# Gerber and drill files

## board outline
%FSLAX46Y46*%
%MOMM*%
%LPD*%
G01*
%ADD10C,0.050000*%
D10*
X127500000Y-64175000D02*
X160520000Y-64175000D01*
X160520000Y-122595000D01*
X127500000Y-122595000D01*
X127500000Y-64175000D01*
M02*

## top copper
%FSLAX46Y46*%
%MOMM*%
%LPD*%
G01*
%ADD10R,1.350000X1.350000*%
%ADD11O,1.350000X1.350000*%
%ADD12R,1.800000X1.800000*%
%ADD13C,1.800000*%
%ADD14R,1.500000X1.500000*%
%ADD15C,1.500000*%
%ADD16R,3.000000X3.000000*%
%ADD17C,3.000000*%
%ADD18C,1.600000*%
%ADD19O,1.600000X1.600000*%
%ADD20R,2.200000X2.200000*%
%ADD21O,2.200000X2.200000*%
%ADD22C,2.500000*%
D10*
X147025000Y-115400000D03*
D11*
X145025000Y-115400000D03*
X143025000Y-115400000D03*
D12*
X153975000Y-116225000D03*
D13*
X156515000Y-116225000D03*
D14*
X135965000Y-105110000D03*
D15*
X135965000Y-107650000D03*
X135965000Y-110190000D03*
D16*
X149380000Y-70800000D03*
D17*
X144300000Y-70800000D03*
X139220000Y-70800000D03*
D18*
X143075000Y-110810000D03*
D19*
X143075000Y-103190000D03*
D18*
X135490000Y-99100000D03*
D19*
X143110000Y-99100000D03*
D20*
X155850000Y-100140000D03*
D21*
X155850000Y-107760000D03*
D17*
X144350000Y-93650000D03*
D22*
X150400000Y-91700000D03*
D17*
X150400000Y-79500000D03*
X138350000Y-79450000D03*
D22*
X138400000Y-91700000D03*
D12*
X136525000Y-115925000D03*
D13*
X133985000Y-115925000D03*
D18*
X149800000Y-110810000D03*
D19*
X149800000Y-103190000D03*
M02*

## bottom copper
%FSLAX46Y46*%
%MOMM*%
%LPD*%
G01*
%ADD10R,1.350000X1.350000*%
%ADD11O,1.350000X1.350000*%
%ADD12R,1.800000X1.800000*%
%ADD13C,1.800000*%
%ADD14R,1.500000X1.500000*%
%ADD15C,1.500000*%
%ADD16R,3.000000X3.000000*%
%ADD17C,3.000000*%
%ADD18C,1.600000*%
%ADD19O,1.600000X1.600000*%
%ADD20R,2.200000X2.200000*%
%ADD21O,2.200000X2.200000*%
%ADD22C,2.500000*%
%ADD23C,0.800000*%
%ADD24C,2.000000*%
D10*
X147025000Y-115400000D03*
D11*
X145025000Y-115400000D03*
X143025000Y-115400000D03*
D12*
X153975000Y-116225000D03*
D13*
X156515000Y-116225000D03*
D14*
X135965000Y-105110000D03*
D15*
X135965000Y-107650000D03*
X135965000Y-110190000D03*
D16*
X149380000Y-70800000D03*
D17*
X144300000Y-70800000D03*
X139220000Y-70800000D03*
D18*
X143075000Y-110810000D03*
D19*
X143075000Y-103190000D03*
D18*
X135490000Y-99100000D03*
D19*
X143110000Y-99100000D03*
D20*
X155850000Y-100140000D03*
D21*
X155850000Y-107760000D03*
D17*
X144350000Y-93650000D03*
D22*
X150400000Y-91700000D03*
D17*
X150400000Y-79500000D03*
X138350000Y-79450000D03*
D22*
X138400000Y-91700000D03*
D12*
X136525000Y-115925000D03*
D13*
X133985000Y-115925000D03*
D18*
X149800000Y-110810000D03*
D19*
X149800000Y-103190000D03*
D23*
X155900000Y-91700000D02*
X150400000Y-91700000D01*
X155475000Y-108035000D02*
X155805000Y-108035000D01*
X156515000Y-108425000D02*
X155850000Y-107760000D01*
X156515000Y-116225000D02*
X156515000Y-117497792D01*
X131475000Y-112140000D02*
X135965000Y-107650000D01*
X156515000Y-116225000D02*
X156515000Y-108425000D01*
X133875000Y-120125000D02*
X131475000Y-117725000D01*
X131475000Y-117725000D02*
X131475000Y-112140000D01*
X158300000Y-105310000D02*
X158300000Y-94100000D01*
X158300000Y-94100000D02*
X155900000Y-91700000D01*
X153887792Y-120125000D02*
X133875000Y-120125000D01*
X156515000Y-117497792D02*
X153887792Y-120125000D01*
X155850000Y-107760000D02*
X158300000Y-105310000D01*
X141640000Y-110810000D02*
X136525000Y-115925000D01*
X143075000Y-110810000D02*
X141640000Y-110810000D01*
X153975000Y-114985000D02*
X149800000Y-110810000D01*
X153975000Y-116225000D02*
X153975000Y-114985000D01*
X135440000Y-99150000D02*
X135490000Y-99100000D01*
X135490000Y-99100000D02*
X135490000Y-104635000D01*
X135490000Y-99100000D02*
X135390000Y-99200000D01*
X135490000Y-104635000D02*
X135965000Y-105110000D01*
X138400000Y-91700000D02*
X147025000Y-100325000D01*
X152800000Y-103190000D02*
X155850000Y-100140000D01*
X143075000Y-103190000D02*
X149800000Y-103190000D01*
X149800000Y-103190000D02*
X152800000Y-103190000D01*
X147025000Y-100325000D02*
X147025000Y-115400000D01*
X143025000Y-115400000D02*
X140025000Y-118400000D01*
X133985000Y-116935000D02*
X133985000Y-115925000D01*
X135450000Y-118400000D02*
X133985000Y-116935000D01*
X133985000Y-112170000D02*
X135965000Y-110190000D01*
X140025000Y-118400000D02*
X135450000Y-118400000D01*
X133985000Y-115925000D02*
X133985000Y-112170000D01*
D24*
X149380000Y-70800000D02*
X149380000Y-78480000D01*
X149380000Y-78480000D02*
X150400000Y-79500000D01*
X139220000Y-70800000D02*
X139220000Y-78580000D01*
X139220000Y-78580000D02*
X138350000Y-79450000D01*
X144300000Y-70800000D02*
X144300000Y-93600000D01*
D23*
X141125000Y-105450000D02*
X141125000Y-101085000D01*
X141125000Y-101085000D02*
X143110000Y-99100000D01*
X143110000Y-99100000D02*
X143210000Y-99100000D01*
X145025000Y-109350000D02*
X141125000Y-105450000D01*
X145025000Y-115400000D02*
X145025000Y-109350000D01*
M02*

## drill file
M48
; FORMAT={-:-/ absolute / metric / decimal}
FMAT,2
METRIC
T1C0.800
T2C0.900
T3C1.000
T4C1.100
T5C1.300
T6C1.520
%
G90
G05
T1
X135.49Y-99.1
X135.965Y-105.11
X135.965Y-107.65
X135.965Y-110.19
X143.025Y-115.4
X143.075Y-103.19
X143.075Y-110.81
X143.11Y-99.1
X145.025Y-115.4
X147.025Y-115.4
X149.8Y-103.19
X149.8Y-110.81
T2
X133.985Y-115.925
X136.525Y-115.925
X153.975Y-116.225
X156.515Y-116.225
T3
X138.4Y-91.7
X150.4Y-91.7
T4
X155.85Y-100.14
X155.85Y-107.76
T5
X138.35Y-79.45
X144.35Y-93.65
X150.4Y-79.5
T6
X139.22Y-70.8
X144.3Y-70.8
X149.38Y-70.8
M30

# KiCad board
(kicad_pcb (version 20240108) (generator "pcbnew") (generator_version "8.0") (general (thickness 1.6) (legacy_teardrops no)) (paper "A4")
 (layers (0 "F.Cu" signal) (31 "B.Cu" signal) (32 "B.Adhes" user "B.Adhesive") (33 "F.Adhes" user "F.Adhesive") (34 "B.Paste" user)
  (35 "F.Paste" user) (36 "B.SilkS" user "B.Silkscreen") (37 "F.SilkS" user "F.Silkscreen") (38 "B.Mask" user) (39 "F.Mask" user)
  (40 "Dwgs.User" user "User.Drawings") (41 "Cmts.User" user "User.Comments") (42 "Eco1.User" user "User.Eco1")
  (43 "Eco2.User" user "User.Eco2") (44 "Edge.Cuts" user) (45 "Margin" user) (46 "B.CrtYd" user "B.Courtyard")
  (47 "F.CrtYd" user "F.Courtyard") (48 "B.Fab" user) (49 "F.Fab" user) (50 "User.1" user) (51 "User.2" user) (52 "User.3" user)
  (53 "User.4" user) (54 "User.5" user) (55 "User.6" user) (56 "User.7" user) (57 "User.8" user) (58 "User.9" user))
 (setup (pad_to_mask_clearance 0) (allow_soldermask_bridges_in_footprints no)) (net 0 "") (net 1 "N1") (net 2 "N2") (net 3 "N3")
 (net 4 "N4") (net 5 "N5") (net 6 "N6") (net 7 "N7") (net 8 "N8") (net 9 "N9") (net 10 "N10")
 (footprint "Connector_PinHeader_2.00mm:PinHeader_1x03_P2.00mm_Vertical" (layer "F.Cu") (at 147.025 115.4 -90)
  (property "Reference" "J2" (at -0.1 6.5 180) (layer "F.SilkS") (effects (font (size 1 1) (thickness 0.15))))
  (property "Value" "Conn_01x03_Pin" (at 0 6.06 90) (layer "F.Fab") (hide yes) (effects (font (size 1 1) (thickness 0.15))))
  (pad "1" thru_hole rect (at 0 0 270) (size 1.35 1.35) (drill 0.8) (layers "*.Cu" "*.Mask") (remove_unused_layers no) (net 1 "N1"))
  (pad "2" thru_hole oval (at 0 2 270) (size 1.35 1.35) (drill 0.8) (layers "*.Cu" "*.Mask") (remove_unused_layers no) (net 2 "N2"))
  (pad "3" thru_hole oval (at 0 4 270) (size 1.35 1.35) (drill 0.8) (layers "*.Cu" "*.Mask") (remove_unused_layers no) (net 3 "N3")))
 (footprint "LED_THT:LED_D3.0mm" (layer "F.Cu") (at 153.975 116.225)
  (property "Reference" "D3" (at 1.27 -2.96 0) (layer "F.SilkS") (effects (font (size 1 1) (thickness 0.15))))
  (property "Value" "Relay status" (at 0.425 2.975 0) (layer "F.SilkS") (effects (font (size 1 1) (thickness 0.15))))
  (pad "1" thru_hole rect (at 0 0) (size 1.8 1.8) (drill 0.9) (layers "*.Cu" "*.Mask") (remove_unused_layers no) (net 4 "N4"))
  (pad "2" thru_hole circle (at 2.54 0) (size 1.8 1.8) (drill 0.9) (layers "*.Cu" "*.Mask") (remove_unused_layers no) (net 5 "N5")))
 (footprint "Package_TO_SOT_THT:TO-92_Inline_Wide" (layer "F.Cu") (at 135.965 105.11 -90)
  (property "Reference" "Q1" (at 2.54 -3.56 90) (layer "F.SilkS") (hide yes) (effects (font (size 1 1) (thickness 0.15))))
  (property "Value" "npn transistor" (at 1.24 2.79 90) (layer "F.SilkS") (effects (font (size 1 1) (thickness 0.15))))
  (pad "1" thru_hole rect (at 0 0 270) (size 1.5 1.5) (drill 0.8) (layers "*.Cu" "*.Mask") (remove_unused_layers no) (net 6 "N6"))
  (pad "2" thru_hole circle (at 2.54 0 270) (size 1.5 1.5) (drill 0.8) (layers "*.Cu" "*.Mask") (remove_unused_layers no) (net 5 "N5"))
  (pad "3" thru_hole circle (at 5.08 0 270) (size 1.5 1.5) (drill 0.8) (layers "*.Cu" "*.Mask") (remove_unused_layers no) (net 3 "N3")))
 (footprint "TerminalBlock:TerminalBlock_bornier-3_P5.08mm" (layer "F.Cu") (at 149.38 70.8 180)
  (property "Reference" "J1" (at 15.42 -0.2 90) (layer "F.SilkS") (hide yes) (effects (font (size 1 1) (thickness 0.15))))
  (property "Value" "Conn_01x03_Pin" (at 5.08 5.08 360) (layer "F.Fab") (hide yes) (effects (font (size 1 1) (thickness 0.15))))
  (pad "1" thru_hole rect (at 0 0 180) (size 3 3) (drill 1.52) (layers "*.Cu" "*.Mask") (remove_unused_layers no) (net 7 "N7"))
  (pad "2" thru_hole circle (at 5.08 0 180) (size 3 3) (drill 1.52) (layers "*.Cu" "*.Mask") (remove_unused_layers no) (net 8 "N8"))
  (pad "3" thru_hole circle (at 10.16 0 180) (size 3 3) (drill 1.52) (layers "*.Cu" "*.Mask") (remove_unused_layers no) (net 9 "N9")))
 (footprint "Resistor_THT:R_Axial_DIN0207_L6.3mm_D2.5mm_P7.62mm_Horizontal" (layer "F.Cu") (at 143.075 110.81 90)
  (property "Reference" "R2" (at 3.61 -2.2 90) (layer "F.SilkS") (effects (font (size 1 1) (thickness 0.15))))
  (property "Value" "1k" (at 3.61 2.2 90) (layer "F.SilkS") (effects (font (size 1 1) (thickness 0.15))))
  (pad "1" thru_hole circle (at 0 0 90) (size 1.6 1.6) (drill 0.8) (layers "*.Cu" "*.Mask") (remove_unused_layers no) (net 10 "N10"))
  (pad "2" thru_hole oval (at 7.62 0 90) (size 1.6 1.6) (drill 0.8) (layers "*.Cu" "*.Mask") (remove_unused_layers no) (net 1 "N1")))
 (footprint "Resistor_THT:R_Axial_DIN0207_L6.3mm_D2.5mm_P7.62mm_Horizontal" (layer "F.Cu") (at 135.49 99.1)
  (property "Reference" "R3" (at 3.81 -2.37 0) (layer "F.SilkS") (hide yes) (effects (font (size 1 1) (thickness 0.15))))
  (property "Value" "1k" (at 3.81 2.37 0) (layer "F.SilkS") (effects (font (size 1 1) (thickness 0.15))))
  (pad "1" thru_hole circle (at 0 0) (size 1.6 1.6) (drill 0.8) (layers "*.Cu" "*.Mask") (remove_unused_layers no) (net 6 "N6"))
  (pad "2" thru_hole oval (at 7.62 0) (size 1.6 1.6) (drill 0.8) (layers "*.Cu" "*.Mask") (remove_unused_layers no) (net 2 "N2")))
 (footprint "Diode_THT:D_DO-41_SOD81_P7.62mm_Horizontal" (layer "F.Cu") (at 155.85 100.14 -90)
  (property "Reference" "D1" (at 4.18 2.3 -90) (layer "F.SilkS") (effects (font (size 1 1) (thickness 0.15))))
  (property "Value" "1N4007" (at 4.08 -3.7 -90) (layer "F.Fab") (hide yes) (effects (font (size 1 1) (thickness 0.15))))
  (pad "1" thru_hole rect (at 0 0 270) (size 2.2 2.2) (drill 1.1) (layers "*.Cu" "*.Mask") (remove_unused_layers no) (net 1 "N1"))
  (pad "2" thru_hole oval (at 7.62 0 270) (size 2.2 2.2) (drill 1.1) (layers "*.Cu" "*.Mask") (remove_unused_layers no) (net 5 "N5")))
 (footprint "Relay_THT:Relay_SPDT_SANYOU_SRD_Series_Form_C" (layer "F.Cu") (at 144.35 93.65 90)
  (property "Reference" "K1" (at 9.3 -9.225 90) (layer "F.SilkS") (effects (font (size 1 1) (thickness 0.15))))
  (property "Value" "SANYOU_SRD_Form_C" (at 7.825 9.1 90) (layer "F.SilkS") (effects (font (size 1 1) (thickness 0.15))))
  (pad "1" thru_hole circle (at 0 0 180) (size 3 3) (drill 1.3) (layers "*.Cu" "*.Mask") (remove_unused_layers no) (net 8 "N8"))
  (pad "2" thru_hole circle (at 1.95 6.05 180) (size 2.5 2.5) (drill 1) (layers "*.Cu" "*.Mask") (remove_unused_layers no) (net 5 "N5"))
  (pad "3" thru_hole circle (at 14.15 6.05 180) (size 3 3) (drill 1.3) (layers "*.Cu" "*.Mask") (remove_unused_layers no) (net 7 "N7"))
  (pad "4" thru_hole circle (at 14.2 -6 180) (size 3 3) (drill 1.3) (layers "*.Cu" "*.Mask") (remove_unused_layers no) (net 9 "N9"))
  (pad "5" thru_hole circle (at 1.95 -5.95 180) (size 2.5 2.5) (drill 1) (layers "*.Cu" "*.Mask") (remove_unused_layers no) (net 1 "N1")))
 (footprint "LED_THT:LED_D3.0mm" (layer "F.Cu") (at 136.525 115.925 180)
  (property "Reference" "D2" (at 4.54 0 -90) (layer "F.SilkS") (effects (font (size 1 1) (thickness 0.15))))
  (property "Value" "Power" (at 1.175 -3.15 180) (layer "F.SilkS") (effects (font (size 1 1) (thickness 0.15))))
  (pad "1" thru_hole rect (at 0 0 180) (size 1.8 1.8) (drill 0.9) (layers "*.Cu" "*.Mask") (remove_unused_layers no) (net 10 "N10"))
  (pad "2" thru_hole circle (at 2.54 0 180) (size 1.8 1.8) (drill 0.9) (layers "*.Cu" "*.Mask") (remove_unused_layers no) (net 3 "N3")))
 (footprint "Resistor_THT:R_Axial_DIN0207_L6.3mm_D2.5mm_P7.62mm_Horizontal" (layer "F.Cu") (at 149.8 110.81 90)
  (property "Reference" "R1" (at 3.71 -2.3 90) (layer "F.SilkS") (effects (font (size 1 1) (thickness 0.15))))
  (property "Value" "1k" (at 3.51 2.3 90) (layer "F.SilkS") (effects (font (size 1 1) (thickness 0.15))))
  (pad "1" thru_hole circle (at 0 0 90) (size 1.6 1.6) (drill 0.8) (layers "*.Cu" "*.Mask") (remove_unused_layers no) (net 4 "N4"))
  (pad "2" thru_hole oval (at 7.62 0 90) (size 1.6 1.6) (drill 0.8) (layers "*.Cu" "*.Mask") (remove_unused_layers no) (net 1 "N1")))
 (gr_rect (start 127.5 64.175) (end 160.52 122.595) (stroke (width 0.05) (type default)) (fill none) (layer "Edge.Cuts"))
 (segment (start 155.9 91.7) (end 150.4 91.7) (width 0.8) (layer "B.Cu") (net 5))
 (segment (start 155.475 108.035) (end 155.805 108.035) (width 0.8) (layer "B.Cu") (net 5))
 (segment (start 156.515 108.425) (end 155.85 107.76) (width 0.8) (layer "B.Cu") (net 5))
 (segment (start 156.515 116.225) (end 156.515 117.497792) (width 0.8) (layer "B.Cu") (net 5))
 (segment (start 131.475 112.14) (end 135.965 107.65) (width 0.8) (layer "B.Cu") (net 5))
 (segment (start 156.515 116.225) (end 156.515 108.425) (width 0.8) (layer "B.Cu") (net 5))
 (segment (start 133.875 120.125) (end 131.475 117.725) (width 0.8) (layer "B.Cu") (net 5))
 (segment (start 131.475 117.725) (end 131.475 112.14) (width 0.8) (layer "B.Cu") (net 5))
 (segment (start 158.3 105.31) (end 158.3 94.1) (width 0.8) (layer "B.Cu") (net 5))
 (segment (start 158.3 94.1) (end 155.9 91.7) (width 0.8) (layer "B.Cu") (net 5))
 (segment (start 153.887792 120.125) (end 133.875 120.125) (width 0.8) (layer "B.Cu") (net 5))
 (segment (start 156.515 117.497792) (end 153.887792 120.125) (width 0.8) (layer "B.Cu") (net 5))
 (segment (start 155.85 107.76) (end 158.3 105.31) (width 0.8) (layer "B.Cu") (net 5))
 (segment (start 141.64 110.81) (end 136.525 115.925) (width 0.8) (layer "B.Cu") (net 10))
 (segment (start 143.075 110.81) (end 141.64 110.81) (width 0.8) (layer "B.Cu") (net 10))
 (segment (start 153.975 114.985) (end 149.8 110.81) (width 0.8) (layer "B.Cu") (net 4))
 (segment (start 153.975 116.225) (end 153.975 114.985) (width 0.8) (layer "B.Cu") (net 4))
 (segment (start 135.44 99.15) (end 135.49 99.1) (width 0.8) (layer "B.Cu") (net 6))
 (segment (start 135.49 99.1) (end 135.49 104.635) (width 0.8) (layer "B.Cu") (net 6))
 (segment (start 135.49 99.1) (end 135.39 99.2) (width 0.8) (layer "B.Cu") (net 6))
 (segment (start 135.49 104.635) (end 135.965 105.11) (width 0.8) (layer "B.Cu") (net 6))
 (segment (start 138.4 91.7) (end 147.025 100.325) (width 0.8) (layer "B.Cu") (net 1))
 (segment (start 152.8 103.19) (end 155.85 100.14) (width 0.8) (layer "B.Cu") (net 1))
 (segment (start 143.075 103.19) (end 149.8 103.19) (width 0.8) (layer "B.Cu") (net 1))
 (segment (start 149.8 103.19) (end 152.8 103.19) (width 0.8) (layer "B.Cu") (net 1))
 (segment (start 147.025 100.325) (end 147.025 115.4) (width 0.8) (layer "B.Cu") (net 1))
 (segment (start 143.025 115.4) (end 140.025 118.4) (width 0.8) (layer "B.Cu") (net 3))
 (segment (start 133.985 116.935) (end 133.985 115.925) (width 0.8) (layer "B.Cu") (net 3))
 (segment (start 135.45 118.4) (end 133.985 116.935) (width 0.8) (layer "B.Cu") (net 3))
 (segment (start 133.985 112.17) (end 135.965 110.19) (width 0.8) (layer "B.Cu") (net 3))
 (segment (start 140.025 118.4) (end 135.45 118.4) (width 0.8) (layer "B.Cu") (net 3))
 (segment (start 133.985 115.925) (end 133.985 112.17) (width 0.8) (layer "B.Cu") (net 3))
 (segment (start 149.38 70.8) (end 149.38 78.48) (width 2) (layer "B.Cu") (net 7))
 (segment (start 149.38 78.48) (end 150.4 79.5) (width 2) (layer "B.Cu") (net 7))
 (segment (start 139.22 70.8) (end 139.22 78.58) (width 2) (layer "B.Cu") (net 9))
 (segment (start 139.22 78.58) (end 138.35 79.45) (width 2) (layer "B.Cu") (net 9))
 (segment (start 144.3 70.8) (end 144.3 93.6) (width 2) (layer "B.Cu") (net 8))
 (segment (start 141.125 105.45) (end 141.125 101.085) (width 0.8) (layer "B.Cu") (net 2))
 (segment (start 141.125 101.085) (end 143.11 99.1) (width 0.8) (layer "B.Cu") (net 2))
 (segment (start 143.11 99.1) (end 143.21 99.1) (width 0.8) (layer "B.Cu") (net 2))
 (segment (start 145.025 109.35) (end 141.125 105.45) (width 0.8) (layer "B.Cu") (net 2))
 (segment (start 145.025 115.4) (end 145.025 109.35) (width 0.8) (layer "B.Cu") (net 2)))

